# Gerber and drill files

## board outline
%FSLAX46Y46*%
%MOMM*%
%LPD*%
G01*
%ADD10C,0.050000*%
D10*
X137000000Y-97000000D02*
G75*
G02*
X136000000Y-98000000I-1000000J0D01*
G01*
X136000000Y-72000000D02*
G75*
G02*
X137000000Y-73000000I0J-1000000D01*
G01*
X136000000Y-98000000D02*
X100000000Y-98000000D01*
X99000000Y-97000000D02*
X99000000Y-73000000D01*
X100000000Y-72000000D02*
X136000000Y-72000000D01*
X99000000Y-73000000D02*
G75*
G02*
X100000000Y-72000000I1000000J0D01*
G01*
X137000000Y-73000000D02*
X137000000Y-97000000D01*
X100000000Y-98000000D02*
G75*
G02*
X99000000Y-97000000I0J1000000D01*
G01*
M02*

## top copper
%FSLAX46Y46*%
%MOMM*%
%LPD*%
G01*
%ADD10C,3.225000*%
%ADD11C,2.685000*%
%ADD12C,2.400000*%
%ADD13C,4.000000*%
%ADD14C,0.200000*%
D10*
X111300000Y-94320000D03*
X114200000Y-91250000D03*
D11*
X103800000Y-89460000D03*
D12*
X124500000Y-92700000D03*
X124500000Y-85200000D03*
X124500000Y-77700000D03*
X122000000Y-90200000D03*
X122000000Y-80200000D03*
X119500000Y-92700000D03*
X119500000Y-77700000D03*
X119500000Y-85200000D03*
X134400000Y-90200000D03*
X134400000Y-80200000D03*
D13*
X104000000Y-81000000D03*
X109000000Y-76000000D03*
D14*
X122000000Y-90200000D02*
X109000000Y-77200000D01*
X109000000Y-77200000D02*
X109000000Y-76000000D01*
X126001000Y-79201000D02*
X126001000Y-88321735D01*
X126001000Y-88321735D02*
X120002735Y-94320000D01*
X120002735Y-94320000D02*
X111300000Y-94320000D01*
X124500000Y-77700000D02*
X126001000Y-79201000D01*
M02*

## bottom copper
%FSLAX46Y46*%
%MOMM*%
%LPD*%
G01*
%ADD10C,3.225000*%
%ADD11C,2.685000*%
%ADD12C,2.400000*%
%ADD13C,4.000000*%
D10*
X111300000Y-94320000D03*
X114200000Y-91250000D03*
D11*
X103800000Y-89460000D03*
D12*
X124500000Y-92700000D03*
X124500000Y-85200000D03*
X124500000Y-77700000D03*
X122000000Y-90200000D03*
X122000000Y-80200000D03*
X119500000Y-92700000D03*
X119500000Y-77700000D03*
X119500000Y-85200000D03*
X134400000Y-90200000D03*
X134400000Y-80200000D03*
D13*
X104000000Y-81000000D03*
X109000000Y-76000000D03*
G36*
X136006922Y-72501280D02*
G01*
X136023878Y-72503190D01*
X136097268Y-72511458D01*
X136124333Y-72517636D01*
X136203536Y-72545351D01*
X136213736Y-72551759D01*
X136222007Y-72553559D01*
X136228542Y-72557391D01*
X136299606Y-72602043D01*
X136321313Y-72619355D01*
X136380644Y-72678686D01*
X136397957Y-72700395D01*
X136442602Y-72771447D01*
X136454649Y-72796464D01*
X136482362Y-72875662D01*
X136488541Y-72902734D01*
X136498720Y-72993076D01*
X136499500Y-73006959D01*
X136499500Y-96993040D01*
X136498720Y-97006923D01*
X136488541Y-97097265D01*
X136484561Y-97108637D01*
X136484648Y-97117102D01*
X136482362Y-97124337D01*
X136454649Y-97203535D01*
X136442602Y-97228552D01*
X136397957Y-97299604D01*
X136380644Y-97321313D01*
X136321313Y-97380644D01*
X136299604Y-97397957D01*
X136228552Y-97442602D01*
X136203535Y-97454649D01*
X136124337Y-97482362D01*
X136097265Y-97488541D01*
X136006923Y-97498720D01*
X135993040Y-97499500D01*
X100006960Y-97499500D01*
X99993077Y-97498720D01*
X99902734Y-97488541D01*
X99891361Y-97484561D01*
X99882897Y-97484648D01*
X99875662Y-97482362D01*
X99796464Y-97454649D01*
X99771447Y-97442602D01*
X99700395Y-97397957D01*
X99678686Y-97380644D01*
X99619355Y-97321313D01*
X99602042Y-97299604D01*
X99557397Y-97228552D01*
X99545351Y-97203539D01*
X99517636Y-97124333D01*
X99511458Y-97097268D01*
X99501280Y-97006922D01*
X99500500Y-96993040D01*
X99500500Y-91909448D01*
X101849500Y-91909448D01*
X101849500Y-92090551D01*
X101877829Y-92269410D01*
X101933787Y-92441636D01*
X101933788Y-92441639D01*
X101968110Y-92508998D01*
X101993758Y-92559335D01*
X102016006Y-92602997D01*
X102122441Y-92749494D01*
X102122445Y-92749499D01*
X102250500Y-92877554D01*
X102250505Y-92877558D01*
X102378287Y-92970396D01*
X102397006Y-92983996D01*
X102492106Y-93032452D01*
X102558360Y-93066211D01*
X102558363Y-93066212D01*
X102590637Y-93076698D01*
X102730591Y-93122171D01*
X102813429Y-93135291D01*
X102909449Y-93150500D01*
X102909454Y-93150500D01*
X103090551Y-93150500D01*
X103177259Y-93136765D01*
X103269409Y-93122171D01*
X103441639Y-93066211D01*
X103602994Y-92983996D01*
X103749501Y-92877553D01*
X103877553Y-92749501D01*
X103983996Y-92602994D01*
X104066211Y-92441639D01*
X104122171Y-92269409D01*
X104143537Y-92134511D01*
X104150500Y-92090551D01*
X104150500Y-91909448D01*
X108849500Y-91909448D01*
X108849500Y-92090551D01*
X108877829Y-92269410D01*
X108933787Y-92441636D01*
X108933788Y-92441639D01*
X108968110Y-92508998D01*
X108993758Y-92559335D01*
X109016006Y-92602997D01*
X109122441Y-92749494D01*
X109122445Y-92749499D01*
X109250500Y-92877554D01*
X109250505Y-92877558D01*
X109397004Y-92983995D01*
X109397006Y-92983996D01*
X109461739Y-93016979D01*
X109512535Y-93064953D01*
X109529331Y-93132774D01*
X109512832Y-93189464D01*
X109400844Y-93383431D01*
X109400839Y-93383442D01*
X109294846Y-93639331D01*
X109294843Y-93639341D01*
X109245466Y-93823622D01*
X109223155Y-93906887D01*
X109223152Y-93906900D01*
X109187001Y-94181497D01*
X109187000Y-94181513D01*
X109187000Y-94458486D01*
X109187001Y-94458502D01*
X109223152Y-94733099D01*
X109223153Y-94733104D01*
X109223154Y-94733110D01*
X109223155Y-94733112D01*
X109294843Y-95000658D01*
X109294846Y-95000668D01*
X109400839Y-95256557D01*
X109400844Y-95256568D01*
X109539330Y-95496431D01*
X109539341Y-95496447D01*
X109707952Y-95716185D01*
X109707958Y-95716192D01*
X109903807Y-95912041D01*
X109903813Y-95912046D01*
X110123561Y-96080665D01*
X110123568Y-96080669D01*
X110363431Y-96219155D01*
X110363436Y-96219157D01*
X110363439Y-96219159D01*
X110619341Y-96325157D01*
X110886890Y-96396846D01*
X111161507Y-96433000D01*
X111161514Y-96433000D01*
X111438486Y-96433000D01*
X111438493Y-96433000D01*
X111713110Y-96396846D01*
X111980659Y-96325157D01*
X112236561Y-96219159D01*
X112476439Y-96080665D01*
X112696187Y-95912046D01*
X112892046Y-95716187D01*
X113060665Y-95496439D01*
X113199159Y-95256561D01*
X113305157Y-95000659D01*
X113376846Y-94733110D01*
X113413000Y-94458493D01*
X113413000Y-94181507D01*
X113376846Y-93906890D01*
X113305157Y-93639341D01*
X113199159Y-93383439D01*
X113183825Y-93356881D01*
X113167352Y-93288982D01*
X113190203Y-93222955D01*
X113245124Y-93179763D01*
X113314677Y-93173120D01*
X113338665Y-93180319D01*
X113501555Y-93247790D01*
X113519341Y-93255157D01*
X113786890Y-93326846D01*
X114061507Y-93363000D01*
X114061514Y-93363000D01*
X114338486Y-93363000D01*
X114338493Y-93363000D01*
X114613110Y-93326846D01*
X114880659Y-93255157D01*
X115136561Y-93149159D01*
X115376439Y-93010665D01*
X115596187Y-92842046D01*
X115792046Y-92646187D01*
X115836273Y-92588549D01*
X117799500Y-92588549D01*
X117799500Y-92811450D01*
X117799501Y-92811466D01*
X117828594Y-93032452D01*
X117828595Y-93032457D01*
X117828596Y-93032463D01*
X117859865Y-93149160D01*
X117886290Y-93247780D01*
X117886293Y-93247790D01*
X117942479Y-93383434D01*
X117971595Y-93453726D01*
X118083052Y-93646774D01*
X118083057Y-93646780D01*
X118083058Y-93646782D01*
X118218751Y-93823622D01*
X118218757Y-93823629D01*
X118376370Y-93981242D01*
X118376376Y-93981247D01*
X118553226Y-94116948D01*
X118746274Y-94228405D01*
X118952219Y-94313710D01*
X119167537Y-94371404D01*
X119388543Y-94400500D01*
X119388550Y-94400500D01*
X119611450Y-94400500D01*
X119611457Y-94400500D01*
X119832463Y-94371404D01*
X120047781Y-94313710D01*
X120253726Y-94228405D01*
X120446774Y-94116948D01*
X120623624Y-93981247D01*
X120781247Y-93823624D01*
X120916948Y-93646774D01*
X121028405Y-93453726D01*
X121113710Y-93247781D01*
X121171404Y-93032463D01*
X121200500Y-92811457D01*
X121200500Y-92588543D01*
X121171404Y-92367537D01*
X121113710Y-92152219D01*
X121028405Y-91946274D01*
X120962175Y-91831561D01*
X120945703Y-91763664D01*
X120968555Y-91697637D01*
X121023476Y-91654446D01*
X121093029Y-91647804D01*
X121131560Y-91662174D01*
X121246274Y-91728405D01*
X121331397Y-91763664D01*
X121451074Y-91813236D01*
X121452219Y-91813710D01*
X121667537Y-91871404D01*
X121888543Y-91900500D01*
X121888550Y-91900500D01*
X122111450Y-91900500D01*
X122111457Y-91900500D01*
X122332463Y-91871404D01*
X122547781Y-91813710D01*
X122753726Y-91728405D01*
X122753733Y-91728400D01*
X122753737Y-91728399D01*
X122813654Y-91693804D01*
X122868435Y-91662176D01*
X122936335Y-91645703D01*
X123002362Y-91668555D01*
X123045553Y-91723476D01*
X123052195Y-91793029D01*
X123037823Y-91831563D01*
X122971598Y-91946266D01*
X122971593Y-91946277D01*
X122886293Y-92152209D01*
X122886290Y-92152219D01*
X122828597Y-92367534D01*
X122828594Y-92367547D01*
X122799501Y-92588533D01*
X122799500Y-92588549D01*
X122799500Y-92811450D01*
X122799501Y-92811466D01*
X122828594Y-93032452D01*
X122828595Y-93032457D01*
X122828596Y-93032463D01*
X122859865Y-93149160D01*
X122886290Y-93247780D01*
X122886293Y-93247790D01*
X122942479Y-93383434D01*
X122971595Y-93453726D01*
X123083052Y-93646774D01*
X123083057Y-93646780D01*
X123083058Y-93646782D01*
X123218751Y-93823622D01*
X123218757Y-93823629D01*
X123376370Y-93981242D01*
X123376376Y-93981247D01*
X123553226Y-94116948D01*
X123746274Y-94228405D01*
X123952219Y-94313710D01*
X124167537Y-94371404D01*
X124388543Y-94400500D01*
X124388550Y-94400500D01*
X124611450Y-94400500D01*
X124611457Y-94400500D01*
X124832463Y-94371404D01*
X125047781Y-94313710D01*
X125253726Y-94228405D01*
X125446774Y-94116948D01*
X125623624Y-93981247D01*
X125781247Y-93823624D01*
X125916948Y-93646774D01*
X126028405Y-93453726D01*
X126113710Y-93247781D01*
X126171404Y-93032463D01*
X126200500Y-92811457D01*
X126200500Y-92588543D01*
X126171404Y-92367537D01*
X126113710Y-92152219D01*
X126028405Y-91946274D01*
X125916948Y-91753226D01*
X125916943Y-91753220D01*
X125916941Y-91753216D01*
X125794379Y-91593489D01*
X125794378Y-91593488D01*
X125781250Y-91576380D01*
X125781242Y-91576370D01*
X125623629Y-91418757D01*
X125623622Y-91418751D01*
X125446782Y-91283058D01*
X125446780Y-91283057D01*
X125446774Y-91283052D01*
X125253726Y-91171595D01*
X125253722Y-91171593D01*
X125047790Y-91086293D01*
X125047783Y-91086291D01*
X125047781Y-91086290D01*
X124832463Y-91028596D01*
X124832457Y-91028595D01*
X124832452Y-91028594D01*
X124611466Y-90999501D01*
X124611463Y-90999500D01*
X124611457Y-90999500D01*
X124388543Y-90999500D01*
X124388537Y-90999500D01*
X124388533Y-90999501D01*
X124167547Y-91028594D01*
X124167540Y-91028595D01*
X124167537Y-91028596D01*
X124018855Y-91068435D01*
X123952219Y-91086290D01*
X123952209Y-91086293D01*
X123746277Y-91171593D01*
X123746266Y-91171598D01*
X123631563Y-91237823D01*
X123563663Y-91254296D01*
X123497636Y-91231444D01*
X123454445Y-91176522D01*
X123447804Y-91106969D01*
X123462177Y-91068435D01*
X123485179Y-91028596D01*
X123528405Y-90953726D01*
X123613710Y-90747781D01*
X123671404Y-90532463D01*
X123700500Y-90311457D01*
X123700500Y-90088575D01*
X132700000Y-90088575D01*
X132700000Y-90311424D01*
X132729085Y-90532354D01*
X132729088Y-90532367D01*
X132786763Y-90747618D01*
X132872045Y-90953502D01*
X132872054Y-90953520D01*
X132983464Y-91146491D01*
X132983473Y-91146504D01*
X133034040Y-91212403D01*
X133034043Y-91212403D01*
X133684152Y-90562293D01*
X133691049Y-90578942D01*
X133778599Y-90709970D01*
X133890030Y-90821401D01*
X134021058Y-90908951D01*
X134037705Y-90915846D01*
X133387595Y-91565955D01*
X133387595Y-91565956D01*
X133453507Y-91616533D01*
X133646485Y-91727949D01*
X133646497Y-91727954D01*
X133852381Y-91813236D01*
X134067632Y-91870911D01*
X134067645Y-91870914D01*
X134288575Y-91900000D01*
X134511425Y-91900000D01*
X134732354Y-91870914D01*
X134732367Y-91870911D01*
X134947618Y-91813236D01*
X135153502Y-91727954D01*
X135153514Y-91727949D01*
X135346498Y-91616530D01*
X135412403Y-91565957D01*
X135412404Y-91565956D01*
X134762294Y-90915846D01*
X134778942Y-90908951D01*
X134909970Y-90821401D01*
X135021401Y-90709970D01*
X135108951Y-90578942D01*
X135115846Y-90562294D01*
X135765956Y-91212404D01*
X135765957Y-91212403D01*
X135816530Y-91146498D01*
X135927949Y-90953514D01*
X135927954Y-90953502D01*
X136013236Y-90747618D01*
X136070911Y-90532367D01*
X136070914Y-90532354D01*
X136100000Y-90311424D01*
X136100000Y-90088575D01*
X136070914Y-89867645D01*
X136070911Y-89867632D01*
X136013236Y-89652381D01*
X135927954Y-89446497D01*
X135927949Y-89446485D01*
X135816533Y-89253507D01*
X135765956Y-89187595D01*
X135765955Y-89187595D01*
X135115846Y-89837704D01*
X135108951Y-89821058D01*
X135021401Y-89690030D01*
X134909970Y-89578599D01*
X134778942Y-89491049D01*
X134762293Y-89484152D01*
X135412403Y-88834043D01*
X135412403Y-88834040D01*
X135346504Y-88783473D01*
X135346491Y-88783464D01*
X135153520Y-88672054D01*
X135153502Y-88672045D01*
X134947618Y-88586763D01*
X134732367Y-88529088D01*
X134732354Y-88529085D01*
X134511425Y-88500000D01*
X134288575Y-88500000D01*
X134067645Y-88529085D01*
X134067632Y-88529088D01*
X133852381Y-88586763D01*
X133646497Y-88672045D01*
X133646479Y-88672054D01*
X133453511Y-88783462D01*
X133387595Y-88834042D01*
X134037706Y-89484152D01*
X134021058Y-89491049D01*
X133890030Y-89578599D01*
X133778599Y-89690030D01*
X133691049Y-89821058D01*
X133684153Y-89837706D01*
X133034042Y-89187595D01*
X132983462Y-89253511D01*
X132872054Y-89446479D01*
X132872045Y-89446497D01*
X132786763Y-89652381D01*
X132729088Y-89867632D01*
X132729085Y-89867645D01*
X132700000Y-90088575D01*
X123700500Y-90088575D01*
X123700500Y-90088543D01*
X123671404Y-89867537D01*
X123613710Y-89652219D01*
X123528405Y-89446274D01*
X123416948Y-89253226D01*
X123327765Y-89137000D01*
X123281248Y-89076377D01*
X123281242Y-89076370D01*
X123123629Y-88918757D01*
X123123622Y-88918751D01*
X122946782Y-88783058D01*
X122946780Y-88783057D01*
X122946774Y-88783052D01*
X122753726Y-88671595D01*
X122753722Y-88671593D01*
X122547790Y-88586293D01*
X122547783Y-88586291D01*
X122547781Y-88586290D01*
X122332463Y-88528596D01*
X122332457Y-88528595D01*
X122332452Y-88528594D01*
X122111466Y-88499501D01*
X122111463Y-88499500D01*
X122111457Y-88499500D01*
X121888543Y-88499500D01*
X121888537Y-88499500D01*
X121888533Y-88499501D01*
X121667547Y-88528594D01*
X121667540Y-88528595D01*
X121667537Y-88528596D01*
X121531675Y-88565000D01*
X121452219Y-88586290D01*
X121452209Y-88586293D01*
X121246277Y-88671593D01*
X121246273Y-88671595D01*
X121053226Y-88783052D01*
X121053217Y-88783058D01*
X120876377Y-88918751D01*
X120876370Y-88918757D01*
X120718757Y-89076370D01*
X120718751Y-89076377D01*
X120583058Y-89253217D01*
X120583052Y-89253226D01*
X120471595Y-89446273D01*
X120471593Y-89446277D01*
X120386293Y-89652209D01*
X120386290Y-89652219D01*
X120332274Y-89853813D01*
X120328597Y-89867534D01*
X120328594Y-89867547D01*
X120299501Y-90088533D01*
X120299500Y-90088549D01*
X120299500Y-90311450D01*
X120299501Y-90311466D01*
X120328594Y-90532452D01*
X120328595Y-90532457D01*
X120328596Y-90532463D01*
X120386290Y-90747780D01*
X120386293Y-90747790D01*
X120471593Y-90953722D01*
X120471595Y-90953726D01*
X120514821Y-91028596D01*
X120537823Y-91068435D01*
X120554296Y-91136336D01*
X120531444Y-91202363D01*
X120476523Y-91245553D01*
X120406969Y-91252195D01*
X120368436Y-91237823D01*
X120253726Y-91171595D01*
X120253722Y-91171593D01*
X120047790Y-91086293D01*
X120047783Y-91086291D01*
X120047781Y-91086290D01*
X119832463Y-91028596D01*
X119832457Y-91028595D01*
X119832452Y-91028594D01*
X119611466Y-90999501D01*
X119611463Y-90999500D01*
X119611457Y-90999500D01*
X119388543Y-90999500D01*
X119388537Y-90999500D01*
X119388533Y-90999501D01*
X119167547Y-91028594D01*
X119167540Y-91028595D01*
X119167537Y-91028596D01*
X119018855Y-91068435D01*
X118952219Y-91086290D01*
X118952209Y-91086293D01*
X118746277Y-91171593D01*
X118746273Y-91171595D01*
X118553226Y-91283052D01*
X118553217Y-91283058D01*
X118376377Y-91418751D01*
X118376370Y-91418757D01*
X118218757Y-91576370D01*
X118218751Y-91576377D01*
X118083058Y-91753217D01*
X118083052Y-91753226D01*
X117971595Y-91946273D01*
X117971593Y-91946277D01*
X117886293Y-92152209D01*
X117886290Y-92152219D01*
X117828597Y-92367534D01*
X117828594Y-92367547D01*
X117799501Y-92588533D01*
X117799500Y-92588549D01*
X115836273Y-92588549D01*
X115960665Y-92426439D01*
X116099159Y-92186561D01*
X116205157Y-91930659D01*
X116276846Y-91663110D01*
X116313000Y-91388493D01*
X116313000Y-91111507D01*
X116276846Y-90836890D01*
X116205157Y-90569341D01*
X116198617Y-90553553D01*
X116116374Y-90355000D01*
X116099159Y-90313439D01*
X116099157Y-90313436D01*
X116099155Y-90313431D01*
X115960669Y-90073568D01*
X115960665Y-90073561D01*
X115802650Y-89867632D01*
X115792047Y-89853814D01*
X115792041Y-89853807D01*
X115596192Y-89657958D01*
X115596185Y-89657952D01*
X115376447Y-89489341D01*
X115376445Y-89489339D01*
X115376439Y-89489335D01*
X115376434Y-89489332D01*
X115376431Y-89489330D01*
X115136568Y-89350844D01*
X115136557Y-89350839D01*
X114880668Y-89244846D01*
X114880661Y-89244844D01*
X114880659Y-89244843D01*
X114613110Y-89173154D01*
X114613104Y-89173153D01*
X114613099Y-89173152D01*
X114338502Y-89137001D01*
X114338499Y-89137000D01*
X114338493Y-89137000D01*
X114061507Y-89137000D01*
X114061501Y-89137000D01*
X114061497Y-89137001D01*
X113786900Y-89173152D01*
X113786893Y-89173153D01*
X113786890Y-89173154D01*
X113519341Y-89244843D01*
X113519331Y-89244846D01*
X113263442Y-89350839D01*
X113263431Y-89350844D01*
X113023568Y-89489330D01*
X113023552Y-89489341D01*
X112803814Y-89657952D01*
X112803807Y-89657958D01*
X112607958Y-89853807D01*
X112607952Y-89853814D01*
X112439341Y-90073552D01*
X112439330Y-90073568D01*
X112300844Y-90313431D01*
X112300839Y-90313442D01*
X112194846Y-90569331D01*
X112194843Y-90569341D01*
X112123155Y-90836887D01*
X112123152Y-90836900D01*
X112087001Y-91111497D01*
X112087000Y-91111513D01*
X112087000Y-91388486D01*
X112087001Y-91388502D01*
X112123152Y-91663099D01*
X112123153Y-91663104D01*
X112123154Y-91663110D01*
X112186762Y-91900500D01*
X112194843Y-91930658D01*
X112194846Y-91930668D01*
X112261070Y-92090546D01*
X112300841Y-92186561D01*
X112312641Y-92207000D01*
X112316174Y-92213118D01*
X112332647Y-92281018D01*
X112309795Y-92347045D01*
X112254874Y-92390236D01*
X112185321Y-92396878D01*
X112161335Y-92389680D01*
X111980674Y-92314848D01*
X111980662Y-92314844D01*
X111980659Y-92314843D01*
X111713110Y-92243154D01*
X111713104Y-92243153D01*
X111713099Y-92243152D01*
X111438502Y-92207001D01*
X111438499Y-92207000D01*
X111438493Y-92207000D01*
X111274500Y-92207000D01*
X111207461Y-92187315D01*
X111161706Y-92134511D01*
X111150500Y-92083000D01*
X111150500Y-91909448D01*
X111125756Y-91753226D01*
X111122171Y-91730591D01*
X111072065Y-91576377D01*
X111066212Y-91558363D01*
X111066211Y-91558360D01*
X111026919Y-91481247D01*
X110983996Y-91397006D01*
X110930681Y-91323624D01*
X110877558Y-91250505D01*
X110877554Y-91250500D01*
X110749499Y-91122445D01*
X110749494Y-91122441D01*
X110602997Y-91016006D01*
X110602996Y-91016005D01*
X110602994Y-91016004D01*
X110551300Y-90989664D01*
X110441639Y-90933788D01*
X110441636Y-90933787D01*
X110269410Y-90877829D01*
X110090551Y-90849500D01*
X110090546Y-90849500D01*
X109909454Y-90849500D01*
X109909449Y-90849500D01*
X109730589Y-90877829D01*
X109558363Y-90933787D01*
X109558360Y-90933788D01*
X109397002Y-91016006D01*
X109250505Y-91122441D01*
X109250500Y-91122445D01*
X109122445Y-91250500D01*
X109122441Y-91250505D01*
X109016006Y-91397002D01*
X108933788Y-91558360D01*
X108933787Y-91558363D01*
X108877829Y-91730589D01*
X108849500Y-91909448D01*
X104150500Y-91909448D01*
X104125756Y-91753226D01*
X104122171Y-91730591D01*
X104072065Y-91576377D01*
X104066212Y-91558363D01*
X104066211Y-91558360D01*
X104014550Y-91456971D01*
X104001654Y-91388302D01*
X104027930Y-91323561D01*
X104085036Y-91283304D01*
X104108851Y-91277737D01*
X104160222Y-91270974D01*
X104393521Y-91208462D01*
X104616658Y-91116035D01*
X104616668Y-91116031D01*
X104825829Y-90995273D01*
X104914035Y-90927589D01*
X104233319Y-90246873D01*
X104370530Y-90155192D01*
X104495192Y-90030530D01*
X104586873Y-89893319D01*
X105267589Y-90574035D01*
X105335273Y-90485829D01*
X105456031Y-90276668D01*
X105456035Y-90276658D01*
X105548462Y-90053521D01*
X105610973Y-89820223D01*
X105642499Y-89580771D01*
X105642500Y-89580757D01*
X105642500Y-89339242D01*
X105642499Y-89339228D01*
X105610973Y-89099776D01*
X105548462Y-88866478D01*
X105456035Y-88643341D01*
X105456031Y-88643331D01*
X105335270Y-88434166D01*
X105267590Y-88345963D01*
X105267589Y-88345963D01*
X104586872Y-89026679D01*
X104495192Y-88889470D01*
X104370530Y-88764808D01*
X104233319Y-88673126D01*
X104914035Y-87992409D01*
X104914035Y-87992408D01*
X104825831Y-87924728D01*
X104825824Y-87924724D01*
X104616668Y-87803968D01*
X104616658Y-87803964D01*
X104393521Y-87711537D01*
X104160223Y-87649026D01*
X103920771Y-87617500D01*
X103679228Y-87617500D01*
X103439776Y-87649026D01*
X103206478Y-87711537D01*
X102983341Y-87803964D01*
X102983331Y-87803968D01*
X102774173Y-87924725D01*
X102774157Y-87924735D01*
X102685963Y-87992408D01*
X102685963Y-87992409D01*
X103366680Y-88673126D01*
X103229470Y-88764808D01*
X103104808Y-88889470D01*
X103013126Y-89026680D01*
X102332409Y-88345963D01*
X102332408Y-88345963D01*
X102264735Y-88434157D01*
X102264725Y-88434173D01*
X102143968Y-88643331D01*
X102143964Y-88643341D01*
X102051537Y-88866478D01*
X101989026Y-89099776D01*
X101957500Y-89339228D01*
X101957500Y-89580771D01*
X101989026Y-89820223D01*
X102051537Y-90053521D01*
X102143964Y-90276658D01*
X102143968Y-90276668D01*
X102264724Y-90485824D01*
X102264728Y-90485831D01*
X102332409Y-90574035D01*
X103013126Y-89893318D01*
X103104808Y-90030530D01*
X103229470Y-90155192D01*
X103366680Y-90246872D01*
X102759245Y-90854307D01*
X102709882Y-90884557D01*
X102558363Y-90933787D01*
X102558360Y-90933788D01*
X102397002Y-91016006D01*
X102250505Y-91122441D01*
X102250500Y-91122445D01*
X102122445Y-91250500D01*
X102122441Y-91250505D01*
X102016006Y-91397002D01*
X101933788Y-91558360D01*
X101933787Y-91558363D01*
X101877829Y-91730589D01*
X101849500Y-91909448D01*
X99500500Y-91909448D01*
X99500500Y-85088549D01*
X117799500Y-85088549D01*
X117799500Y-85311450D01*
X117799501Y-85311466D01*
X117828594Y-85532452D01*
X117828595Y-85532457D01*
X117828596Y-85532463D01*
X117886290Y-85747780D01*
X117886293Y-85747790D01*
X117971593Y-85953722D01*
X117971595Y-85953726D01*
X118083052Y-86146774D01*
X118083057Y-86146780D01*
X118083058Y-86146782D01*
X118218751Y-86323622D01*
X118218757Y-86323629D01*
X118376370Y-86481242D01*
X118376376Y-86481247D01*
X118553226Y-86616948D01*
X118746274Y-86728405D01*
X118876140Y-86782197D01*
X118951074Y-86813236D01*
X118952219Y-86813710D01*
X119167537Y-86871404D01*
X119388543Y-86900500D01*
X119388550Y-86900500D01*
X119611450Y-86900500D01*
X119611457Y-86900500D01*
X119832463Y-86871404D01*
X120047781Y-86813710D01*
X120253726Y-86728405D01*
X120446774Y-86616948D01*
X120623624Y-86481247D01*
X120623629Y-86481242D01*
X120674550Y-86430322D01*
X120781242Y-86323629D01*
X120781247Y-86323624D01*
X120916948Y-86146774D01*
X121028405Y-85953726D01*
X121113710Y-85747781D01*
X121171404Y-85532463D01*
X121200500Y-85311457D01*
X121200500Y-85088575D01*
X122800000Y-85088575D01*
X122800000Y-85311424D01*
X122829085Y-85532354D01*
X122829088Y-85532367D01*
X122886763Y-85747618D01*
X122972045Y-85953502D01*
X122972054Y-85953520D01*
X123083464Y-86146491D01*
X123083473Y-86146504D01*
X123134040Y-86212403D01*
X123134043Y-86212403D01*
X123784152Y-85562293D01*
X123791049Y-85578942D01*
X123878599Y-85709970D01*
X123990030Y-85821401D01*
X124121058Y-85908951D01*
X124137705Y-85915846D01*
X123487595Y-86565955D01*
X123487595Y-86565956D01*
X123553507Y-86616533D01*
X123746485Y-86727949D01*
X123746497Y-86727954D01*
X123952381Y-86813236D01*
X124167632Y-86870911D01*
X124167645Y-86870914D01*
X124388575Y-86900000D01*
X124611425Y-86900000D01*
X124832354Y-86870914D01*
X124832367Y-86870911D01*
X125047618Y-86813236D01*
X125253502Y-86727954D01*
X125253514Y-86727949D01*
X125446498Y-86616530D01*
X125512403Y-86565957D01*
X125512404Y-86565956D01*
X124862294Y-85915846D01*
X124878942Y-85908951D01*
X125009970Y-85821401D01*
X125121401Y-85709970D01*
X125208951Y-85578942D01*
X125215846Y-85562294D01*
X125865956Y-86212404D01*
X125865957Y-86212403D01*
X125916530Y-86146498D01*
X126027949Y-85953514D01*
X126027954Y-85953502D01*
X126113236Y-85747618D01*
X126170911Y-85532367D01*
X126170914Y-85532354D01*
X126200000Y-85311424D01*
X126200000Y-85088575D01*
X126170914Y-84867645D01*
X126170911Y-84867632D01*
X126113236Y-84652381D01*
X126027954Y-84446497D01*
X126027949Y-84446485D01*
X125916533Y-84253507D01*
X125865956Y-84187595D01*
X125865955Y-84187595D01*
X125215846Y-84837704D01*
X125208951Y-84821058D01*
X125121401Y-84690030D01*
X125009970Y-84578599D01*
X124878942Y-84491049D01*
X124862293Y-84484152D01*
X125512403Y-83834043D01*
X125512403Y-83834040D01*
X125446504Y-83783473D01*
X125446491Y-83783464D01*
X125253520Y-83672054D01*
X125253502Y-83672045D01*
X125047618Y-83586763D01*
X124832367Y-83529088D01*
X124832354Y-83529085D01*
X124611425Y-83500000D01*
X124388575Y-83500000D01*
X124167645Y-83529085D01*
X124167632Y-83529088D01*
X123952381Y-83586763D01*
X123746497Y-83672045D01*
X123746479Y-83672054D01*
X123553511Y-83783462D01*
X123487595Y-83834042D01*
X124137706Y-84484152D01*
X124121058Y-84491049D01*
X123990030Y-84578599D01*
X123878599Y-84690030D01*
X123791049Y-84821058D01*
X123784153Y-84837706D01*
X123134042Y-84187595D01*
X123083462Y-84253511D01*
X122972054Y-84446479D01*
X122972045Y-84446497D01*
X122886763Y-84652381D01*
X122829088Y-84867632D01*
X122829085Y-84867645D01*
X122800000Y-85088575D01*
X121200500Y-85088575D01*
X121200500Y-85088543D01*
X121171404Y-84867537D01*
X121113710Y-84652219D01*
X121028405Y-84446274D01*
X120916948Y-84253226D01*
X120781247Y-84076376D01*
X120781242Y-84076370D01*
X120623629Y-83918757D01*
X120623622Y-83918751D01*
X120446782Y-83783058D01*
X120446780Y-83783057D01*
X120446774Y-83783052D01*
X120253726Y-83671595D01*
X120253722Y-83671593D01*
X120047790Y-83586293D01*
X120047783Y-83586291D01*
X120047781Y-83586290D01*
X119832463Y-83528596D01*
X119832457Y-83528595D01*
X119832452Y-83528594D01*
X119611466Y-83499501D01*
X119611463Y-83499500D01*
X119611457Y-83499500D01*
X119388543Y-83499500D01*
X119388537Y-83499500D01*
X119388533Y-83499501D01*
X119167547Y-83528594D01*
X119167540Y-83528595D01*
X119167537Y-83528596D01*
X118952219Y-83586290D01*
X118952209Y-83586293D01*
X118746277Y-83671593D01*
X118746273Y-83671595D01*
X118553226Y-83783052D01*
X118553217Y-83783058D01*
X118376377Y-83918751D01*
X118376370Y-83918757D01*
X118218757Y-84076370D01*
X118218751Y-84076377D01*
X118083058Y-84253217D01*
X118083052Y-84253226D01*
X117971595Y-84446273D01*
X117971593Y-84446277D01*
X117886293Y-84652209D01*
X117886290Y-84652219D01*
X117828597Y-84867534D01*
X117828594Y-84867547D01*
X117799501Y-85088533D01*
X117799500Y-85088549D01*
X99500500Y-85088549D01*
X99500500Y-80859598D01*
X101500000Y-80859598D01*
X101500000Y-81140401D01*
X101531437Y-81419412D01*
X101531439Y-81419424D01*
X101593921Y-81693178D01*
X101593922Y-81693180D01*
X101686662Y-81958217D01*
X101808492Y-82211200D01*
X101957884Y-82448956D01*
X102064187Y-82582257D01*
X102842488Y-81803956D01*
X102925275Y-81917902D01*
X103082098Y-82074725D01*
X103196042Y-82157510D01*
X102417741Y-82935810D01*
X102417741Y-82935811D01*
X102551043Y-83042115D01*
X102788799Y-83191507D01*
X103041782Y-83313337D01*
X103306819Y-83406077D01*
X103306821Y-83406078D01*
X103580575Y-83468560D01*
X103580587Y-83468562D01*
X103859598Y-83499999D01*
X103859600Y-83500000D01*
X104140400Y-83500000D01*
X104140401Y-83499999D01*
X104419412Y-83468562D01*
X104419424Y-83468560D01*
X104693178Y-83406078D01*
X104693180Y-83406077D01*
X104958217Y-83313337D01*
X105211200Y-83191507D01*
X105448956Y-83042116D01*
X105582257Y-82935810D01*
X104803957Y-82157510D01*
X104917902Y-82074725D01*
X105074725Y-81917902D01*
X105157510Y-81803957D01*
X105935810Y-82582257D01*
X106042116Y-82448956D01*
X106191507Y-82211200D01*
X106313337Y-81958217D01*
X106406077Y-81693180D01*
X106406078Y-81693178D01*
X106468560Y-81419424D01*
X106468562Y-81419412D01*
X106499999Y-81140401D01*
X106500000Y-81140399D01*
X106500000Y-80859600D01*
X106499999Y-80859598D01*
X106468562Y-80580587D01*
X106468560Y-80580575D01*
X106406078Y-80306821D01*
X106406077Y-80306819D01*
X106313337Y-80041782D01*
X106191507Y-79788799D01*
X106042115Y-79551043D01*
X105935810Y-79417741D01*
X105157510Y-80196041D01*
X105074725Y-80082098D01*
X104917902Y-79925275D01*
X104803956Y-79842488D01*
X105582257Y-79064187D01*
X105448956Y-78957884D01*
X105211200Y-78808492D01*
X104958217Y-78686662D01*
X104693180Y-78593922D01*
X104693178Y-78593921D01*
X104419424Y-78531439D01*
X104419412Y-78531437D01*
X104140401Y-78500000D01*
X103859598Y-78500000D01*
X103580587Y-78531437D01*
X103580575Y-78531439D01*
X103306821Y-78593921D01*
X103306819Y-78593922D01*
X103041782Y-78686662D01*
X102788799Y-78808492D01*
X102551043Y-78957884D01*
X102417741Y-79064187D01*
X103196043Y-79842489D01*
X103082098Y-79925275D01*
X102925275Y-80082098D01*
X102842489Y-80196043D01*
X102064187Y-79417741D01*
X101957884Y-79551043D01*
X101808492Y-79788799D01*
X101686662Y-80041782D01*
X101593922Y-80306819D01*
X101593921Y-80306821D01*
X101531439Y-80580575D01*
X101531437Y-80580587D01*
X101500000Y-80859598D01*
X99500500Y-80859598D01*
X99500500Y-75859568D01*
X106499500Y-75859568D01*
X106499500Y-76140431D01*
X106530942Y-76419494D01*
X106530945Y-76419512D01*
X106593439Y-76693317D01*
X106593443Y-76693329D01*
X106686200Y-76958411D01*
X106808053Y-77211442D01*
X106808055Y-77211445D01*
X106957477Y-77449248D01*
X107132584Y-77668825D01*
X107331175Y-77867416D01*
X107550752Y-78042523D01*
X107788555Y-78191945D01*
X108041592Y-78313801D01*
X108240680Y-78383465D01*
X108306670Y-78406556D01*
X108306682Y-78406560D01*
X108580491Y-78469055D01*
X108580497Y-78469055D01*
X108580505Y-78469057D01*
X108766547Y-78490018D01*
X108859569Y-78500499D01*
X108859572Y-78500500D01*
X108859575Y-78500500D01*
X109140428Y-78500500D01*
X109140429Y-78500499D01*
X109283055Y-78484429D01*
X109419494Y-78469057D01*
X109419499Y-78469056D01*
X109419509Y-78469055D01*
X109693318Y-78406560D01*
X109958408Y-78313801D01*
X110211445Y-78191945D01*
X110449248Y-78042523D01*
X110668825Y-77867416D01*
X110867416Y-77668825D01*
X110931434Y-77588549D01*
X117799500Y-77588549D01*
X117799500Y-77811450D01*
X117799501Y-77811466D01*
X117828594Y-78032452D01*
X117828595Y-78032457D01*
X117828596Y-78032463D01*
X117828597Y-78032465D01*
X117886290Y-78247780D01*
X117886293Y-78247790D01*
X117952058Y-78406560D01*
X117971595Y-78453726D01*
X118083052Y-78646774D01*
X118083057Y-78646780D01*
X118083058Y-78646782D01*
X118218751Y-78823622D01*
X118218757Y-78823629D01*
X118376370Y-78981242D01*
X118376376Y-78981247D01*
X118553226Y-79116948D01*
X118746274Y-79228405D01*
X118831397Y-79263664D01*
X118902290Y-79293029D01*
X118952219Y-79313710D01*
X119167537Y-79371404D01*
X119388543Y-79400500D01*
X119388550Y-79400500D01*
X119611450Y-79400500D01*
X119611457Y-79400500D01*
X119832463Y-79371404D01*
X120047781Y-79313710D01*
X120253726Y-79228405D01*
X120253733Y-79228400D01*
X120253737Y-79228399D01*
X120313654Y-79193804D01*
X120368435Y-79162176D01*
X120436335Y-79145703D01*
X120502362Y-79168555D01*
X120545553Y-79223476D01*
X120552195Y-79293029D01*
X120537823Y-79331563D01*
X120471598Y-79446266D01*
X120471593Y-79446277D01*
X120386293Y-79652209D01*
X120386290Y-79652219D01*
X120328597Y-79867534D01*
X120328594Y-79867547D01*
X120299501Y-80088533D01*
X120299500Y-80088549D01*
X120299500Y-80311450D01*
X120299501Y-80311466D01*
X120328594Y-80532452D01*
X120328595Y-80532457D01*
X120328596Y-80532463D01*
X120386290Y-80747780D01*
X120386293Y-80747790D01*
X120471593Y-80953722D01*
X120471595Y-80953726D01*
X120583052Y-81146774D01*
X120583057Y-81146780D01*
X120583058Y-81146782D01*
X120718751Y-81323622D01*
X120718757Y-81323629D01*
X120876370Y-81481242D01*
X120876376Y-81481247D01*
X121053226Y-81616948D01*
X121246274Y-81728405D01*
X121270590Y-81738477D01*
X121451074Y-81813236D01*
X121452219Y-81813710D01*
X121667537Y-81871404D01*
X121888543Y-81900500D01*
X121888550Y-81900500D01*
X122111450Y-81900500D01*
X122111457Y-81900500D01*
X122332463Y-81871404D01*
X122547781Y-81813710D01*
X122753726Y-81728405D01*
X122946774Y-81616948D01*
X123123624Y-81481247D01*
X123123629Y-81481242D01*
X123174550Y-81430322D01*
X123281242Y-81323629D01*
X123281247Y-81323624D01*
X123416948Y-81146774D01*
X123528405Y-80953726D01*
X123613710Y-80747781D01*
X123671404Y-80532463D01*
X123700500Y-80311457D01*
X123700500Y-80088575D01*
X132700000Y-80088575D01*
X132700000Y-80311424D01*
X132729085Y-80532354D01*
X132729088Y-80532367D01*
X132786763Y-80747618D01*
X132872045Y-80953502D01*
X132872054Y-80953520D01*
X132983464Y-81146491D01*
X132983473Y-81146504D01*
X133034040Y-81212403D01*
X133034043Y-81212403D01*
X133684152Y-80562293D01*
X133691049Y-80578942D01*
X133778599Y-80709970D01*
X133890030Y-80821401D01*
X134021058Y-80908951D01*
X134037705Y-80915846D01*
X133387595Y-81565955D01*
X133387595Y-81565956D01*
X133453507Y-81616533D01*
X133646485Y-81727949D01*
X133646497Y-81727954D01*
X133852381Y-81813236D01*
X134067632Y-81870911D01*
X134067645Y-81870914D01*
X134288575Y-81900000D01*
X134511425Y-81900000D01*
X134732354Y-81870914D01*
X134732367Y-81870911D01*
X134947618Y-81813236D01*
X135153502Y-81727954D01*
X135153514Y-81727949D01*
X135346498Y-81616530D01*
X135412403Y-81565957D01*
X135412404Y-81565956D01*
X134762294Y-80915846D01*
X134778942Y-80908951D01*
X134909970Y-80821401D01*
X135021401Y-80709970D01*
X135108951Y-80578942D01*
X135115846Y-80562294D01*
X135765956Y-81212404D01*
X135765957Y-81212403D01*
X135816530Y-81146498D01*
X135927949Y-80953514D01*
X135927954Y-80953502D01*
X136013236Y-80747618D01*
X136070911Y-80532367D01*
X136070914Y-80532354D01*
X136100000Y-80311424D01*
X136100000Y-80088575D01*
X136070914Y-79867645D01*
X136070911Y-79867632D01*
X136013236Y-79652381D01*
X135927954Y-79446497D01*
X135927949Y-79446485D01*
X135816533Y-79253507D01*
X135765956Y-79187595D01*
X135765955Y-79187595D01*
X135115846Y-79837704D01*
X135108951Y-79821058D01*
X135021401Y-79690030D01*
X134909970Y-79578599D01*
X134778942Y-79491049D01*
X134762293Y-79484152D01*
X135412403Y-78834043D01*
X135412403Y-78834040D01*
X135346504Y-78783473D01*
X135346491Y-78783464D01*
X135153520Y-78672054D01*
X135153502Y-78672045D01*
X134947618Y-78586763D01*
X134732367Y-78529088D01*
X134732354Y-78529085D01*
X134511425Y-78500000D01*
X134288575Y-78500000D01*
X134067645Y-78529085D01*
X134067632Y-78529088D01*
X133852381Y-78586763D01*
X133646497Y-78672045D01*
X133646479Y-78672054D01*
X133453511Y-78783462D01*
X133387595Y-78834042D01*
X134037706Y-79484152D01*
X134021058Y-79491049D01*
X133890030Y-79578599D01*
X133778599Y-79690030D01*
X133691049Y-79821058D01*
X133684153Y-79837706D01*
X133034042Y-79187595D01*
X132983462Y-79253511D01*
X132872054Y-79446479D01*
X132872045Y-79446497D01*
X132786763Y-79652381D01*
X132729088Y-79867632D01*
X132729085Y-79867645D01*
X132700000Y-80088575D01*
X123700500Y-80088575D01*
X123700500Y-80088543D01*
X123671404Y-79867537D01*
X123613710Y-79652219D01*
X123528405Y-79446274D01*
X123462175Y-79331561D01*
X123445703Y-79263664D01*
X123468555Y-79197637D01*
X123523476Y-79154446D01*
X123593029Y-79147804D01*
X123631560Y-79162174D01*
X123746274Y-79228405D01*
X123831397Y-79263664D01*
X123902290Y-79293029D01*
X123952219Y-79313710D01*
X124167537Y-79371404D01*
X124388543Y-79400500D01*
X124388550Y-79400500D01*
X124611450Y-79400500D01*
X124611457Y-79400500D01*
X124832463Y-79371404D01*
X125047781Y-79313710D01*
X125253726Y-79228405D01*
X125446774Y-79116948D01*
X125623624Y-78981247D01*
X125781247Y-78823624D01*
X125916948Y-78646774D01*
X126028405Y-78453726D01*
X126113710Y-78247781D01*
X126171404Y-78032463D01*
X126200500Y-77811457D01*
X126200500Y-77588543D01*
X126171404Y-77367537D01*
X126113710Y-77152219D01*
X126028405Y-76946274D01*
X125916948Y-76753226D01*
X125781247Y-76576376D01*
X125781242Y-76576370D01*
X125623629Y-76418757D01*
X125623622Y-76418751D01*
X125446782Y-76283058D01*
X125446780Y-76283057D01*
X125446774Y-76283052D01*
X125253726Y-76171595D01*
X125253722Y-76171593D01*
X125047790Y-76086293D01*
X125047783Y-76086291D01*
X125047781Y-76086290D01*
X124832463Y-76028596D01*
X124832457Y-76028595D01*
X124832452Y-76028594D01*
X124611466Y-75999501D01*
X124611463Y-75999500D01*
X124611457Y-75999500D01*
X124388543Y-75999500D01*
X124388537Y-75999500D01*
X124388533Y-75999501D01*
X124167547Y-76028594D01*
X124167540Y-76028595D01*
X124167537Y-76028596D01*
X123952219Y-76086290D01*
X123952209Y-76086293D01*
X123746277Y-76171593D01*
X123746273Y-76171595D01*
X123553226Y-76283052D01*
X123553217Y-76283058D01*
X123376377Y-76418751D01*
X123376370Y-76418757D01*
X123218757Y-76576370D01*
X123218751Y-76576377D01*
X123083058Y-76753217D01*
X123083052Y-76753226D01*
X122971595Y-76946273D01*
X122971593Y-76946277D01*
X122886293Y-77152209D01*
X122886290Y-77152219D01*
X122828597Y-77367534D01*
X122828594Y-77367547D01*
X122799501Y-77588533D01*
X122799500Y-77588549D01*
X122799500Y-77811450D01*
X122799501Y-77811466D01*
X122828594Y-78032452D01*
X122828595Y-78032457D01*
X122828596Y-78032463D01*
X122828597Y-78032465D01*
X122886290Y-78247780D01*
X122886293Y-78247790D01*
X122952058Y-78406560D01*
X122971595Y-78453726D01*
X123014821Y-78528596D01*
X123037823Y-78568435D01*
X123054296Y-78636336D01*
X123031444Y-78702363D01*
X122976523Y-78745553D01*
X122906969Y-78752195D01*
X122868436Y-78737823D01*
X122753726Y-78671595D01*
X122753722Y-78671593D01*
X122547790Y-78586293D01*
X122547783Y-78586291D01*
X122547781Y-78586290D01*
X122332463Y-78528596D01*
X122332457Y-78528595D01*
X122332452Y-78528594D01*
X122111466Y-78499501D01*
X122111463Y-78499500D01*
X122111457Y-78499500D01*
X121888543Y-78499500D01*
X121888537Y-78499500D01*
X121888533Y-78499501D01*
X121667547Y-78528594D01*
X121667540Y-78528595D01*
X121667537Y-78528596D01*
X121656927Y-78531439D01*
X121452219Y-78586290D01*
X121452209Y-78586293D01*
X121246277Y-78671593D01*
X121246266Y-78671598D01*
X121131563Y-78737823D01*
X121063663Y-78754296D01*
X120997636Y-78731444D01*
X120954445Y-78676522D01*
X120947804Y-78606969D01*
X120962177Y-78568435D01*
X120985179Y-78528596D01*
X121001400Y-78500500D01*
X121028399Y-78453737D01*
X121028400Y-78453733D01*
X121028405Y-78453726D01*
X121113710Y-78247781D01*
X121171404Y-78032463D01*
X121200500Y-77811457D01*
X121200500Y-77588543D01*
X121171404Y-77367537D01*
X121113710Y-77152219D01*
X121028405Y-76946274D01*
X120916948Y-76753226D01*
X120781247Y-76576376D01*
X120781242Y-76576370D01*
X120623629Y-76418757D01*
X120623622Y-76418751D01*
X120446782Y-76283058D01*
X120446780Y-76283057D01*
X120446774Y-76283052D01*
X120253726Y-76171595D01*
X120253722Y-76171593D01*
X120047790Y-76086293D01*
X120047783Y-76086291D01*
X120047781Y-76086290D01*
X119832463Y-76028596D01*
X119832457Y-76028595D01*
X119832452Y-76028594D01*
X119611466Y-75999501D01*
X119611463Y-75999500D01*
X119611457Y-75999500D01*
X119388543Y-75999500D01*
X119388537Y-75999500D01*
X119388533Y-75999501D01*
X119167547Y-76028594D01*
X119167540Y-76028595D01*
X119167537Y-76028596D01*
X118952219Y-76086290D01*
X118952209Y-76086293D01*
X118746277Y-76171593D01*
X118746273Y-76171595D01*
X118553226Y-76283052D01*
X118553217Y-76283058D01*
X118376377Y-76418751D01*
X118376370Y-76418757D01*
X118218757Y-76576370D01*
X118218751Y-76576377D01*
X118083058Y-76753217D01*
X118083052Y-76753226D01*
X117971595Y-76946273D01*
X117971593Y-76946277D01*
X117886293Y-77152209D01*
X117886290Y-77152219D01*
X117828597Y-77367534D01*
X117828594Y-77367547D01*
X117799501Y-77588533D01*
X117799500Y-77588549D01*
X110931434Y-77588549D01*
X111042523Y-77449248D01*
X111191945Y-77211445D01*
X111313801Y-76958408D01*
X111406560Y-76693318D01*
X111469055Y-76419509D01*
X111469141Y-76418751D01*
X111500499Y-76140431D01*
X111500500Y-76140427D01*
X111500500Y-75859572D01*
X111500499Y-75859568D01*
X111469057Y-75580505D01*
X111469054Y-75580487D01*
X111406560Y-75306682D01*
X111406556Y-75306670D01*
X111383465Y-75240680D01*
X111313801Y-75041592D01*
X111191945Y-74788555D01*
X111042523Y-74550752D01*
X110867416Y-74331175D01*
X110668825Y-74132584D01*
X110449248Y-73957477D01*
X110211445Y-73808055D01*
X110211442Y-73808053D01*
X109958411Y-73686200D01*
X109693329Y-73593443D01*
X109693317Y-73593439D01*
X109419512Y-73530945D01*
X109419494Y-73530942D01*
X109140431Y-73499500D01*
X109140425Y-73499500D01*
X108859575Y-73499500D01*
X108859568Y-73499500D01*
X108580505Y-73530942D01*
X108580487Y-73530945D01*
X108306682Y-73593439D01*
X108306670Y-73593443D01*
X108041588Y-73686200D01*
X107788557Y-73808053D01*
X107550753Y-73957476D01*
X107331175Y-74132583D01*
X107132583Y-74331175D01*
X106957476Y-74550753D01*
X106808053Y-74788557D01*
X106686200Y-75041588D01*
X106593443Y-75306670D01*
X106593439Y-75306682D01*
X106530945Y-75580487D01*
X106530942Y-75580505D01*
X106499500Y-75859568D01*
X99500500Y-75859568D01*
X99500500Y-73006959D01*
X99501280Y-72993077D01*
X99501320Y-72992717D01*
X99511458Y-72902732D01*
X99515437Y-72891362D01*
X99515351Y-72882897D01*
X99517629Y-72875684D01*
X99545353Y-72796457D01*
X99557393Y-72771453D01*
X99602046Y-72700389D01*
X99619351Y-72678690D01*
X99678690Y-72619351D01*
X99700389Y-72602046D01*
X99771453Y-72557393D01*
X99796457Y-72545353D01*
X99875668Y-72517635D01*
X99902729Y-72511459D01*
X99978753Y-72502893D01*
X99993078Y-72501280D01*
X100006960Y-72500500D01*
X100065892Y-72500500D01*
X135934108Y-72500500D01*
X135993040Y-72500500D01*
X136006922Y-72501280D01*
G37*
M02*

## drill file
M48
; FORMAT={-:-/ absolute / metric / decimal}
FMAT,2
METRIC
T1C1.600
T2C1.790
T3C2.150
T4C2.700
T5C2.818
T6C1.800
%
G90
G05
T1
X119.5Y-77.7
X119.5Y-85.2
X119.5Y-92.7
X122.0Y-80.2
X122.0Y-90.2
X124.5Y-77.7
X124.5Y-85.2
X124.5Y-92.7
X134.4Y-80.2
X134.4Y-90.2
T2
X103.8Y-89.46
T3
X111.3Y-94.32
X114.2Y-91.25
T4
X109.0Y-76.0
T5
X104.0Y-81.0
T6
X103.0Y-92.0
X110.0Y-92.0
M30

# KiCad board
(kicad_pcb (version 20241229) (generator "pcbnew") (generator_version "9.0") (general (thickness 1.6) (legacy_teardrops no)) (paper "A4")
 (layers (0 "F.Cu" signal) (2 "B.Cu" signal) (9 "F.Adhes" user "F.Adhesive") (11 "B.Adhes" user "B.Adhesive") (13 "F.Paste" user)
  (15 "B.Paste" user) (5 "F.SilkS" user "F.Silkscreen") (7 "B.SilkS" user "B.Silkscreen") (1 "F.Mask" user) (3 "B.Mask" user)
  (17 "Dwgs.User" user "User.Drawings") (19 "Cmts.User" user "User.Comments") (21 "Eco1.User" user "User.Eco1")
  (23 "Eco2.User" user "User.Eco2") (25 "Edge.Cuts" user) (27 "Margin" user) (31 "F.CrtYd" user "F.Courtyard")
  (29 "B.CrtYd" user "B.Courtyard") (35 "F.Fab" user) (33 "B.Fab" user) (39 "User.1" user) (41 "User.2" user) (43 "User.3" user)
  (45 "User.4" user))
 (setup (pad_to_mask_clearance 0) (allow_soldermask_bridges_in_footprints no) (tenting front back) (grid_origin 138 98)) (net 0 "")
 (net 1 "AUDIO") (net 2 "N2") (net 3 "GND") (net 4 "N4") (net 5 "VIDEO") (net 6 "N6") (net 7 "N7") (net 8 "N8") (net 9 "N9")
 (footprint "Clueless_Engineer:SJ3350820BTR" (layer "F.Cu") (at 111.3 94.32)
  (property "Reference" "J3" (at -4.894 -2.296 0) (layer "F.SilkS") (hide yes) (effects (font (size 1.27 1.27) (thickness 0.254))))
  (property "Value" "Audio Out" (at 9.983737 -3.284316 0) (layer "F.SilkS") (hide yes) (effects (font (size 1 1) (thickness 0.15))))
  (pad "" np_thru_hole circle (at -8.3 -2.32) (size 1.8 1.8) (drill 1.8) (layers "*.Cu" "*.Mask"))
  (pad "" np_thru_hole circle (at -1.3 -2.32) (size 1.8 1.8) (drill 1.8) (layers "*.Cu" "*.Mask"))
  (pad "2" thru_hole circle (at 0 0) (size 3.225 3.225) (drill 2.15) (layers "*.Cu" "*.Mask") (remove_unused_layers no) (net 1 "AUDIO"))
  (pad "3" thru_hole circle (at 2.9 -3.07) (size 3.225 3.225) (drill 2.15) (layers "*.Cu" "*.Mask") (remove_unused_layers no) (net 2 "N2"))
  (pad "5" thru_hole circle (at -7.5 -4.86) (size 2.685 2.685) (drill 1.79) (layers "*.Cu" "*.Mask") (remove_unused_layers no) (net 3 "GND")))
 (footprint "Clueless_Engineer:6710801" (layer "F.Cu") (at 124.5 92.7 -90)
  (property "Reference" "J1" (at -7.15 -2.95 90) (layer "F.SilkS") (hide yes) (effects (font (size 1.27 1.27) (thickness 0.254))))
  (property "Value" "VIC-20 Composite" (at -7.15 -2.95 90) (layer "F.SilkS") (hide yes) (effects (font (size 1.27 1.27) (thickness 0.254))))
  (pad "1" thru_hole circle (at 0 0 270) (size 2.4 2.4) (drill 1.6) (layers "*.Cu" "*.Mask") (remove_unused_layers no) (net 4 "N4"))
  (pad "2" thru_hole circle (at -7.5 0 270) (size 2.4 2.4) (drill 1.6) (layers "*.Cu" "*.Mask") (remove_unused_layers no) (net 3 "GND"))
  (pad "3" thru_hole circle (at -15 0 270) (size 2.4 2.4) (drill 1.6) (layers "*.Cu" "*.Mask") (remove_unused_layers no) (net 1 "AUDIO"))
  (pad "4" thru_hole circle (at -2.5 2.5 270) (size 2.4 2.4) (drill 1.6) (layers "*.Cu" "*.Mask") (remove_unused_layers no) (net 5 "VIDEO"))
  (pad "5" thru_hole circle (at -12.5 2.5 270) (size 2.4 2.4) (drill 1.6) (layers "*.Cu" "*.Mask") (remove_unused_layers no) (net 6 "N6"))
  (pad "6" thru_hole circle (at 0 5 270) (size 2.4 2.4) (drill 1.6) (layers "*.Cu" "*.Mask") (remove_unused_layers no) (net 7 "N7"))
  (pad "7" thru_hole circle (at -15 5 270) (size 2.4 2.4) (drill 1.6) (layers "*.Cu" "*.Mask") (remove_unused_layers no) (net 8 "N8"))
  (pad "8" thru_hole circle (at -7.5 5 270) (size 2.4 2.4) (drill 1.6) (layers "*.Cu" "*.Mask") (remove_unused_layers no) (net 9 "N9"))
  (pad "MH1" thru_hole circle (at -2.5 -9.9 270) (size 2.4 2.4) (drill 1.6) (layers "*.Cu" "*.Mask") (remove_unused_layers no) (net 3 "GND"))
  (pad "MH2" thru_hole circle (at -12.5 -9.9 270) (size 2.4 2.4) (drill 1.6) (layers "*.Cu" "*.Mask") (remove_unused_layers no)
   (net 3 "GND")))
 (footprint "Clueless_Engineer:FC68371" (layer "F.Cu") (at 104 81)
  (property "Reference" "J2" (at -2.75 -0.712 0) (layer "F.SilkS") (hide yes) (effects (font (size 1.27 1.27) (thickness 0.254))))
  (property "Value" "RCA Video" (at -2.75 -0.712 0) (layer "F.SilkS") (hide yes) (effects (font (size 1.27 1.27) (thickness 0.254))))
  (pad "1" thru_hole circle (at 0 0) (size 4 4) (drill 2.818) (layers "*.Cu" "*.Mask") (remove_unused_layers no) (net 3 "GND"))
  (pad "3" thru_hole circle (at 5 -5) (size 4 4) (drill 2.7) (layers "*.Cu" "*.Mask") (remove_unused_layers no) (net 5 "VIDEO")))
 (gr_arc (start 137 97) (mid 136.707107 97.707107) (end 136 98) (stroke (width 0.05) (type default)) (layer "Edge.Cuts"))
 (gr_arc (start 136 72) (mid 136.707107 72.292893) (end 137 73) (stroke (width 0.05) (type default)) (layer "Edge.Cuts"))
 (gr_line (start 136 98) (end 100 98) (stroke (width 0.05) (type default)) (layer "Edge.Cuts"))
 (gr_line (start 99 97) (end 99 73) (stroke (width 0.05) (type default)) (layer "Edge.Cuts"))
 (gr_line (start 100 72) (end 136 72) (stroke (width 0.05) (type default)) (layer "Edge.Cuts"))
 (gr_arc (start 99 73) (mid 99.292893 72.292893) (end 100 72) (stroke (width 0.05) (type default)) (layer "Edge.Cuts"))
 (gr_line (start 137 73) (end 137 97) (stroke (width 0.05) (type default)) (layer "Edge.Cuts"))
 (gr_arc (start 100 98) (mid 99.292893 97.707107) (end 99 97) (stroke (width 0.05) (type default)) (layer "Edge.Cuts"))
 (segment (start 122 90.2) (end 109 77.2) (width 0.2) (layer "F.Cu") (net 5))
 (segment (start 109 77.2) (end 109 76) (width 0.2) (layer "F.Cu") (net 5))
 (segment (start 126.001 79.201) (end 126.001 88.321735) (width 0.2) (layer "F.Cu") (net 1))
 (segment (start 126.001 88.321735) (end 120.002735 94.32) (width 0.2) (layer "F.Cu") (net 1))
 (segment (start 120.002735 94.32) (end 111.3 94.32) (width 0.2) (layer "F.Cu") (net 1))
 (segment (start 124.5 77.7) (end 126.001 79.201) (width 0.2) (layer "F.Cu") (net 1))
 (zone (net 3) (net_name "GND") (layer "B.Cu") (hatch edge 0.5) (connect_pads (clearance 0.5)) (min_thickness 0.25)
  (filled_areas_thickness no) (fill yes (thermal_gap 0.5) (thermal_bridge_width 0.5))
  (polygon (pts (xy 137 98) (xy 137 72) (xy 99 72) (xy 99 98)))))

